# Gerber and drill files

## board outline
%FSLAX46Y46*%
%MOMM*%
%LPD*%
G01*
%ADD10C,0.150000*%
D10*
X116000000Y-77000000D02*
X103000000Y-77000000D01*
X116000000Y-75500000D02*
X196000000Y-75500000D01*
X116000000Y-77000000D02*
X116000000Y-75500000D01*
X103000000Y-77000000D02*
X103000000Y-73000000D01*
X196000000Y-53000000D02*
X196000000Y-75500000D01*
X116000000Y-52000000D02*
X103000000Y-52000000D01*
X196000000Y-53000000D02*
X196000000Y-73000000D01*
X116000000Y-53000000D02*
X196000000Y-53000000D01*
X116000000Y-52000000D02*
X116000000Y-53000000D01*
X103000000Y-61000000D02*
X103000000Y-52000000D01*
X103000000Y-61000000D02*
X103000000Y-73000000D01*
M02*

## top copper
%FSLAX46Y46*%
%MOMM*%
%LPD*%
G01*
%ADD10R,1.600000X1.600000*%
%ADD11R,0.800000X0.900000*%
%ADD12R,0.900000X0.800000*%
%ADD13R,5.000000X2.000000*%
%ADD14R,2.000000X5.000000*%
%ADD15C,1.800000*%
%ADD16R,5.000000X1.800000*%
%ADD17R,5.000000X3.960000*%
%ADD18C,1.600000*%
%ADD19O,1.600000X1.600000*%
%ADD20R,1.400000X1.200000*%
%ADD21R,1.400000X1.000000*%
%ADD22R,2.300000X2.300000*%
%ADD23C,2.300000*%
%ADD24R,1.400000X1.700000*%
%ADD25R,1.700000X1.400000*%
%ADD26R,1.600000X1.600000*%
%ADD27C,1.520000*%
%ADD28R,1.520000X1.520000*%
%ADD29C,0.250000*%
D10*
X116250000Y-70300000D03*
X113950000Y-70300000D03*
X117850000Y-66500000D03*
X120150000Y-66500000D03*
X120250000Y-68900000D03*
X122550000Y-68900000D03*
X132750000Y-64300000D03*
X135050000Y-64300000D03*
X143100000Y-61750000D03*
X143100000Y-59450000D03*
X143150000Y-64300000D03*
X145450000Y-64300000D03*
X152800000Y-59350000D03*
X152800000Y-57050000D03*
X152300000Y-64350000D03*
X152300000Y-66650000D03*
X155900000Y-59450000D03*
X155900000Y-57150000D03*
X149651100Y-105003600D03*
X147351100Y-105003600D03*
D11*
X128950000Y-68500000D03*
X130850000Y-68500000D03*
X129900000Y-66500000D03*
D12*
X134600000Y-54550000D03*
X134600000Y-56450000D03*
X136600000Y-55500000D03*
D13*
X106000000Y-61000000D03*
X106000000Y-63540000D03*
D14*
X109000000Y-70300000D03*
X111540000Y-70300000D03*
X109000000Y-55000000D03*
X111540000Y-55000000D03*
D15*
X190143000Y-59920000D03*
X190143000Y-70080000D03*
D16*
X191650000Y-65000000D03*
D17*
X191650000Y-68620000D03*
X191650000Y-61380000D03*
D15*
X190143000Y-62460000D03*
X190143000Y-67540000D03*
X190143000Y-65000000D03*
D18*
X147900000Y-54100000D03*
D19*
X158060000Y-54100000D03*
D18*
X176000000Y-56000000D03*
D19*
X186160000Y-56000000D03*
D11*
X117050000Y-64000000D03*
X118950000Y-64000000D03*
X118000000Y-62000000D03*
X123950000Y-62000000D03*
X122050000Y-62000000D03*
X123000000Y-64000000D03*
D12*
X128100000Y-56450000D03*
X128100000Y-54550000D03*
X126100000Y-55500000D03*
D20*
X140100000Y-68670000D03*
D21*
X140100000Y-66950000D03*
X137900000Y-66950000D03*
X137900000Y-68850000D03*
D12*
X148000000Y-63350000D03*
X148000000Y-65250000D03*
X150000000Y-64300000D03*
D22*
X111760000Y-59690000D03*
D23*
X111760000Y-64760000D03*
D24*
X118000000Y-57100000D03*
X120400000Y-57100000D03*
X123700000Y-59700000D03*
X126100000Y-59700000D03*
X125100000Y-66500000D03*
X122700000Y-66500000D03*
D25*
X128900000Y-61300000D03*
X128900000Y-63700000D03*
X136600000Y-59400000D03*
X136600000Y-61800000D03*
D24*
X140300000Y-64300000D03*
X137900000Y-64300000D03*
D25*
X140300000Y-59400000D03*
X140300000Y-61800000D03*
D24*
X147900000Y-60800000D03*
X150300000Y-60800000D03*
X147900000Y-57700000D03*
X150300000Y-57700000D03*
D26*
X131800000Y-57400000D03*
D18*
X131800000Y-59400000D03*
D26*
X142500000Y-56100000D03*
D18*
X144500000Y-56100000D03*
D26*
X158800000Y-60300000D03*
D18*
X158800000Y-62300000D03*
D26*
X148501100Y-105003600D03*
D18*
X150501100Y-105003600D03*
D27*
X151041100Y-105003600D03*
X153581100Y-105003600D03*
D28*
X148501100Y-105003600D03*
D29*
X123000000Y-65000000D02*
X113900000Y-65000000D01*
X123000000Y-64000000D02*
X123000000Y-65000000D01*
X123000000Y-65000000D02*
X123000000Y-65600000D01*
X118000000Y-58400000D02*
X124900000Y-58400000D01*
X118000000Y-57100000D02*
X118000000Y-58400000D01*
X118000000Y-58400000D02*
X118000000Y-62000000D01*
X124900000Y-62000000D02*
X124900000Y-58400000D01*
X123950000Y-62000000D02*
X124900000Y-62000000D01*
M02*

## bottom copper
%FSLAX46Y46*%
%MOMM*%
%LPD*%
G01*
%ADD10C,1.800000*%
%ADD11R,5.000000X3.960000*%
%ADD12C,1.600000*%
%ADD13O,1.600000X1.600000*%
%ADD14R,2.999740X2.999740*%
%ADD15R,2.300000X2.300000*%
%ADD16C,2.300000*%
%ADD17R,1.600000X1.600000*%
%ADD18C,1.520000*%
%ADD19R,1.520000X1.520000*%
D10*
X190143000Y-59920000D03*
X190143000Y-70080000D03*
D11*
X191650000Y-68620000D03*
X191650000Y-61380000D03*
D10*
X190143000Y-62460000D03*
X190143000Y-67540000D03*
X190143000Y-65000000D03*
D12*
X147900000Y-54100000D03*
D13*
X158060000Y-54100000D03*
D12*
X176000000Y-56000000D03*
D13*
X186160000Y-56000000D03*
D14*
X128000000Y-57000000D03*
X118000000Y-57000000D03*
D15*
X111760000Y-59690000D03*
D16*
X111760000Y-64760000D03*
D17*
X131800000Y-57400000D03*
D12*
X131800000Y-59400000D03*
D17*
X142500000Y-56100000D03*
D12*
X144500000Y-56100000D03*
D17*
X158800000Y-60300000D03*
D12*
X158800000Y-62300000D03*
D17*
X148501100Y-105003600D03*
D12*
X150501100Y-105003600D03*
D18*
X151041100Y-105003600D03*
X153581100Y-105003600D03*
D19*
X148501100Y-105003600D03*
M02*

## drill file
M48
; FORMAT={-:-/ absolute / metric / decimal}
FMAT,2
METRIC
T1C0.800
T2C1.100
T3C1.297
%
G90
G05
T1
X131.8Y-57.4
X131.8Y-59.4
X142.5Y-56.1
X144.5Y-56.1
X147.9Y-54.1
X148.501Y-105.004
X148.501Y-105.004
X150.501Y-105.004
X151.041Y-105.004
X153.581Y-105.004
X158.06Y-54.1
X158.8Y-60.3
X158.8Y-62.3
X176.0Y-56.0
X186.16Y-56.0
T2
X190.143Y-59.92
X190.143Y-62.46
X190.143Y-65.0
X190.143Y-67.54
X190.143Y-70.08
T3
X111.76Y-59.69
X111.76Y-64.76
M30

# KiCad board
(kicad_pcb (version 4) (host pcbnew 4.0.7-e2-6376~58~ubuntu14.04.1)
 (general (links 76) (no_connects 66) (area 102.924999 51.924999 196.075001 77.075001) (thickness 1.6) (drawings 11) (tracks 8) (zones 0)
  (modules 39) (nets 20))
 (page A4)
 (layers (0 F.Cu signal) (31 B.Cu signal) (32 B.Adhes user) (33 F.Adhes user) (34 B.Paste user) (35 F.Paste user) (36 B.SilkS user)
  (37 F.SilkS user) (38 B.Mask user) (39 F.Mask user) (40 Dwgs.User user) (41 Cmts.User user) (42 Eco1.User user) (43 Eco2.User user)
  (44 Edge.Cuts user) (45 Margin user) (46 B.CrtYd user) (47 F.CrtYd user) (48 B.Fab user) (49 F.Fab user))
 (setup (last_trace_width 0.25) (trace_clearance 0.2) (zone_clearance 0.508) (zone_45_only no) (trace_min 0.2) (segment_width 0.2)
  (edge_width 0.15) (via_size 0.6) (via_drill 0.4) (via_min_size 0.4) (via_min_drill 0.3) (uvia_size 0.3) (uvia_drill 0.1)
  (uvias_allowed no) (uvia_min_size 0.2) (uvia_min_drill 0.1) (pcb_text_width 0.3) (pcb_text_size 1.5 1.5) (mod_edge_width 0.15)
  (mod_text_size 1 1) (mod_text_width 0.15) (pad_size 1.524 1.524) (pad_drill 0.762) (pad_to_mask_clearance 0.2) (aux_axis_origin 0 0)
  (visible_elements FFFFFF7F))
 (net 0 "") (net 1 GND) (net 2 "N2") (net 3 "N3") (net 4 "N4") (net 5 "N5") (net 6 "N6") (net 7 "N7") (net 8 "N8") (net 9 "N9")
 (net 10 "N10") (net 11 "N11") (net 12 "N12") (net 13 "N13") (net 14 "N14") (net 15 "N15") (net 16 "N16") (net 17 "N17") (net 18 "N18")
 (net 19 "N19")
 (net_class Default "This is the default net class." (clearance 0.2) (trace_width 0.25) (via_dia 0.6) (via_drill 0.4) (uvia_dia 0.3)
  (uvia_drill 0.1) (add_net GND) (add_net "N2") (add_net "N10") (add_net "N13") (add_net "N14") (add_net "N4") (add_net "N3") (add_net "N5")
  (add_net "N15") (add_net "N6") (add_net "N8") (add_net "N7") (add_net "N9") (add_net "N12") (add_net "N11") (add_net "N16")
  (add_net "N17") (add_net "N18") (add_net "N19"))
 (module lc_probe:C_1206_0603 (layer F.Cu) (at 115.1 70.3)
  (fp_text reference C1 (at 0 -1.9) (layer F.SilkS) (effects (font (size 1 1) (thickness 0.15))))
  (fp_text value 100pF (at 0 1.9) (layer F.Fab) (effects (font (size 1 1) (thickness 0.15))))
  (pad 2 smd rect (at 1.15 0) (size 1.6 1.6) (layers F.Cu F.Paste F.Mask) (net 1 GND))
  (pad 1 smd rect (at -1.15 0) (size 1.6 1.6) (layers F.Cu F.Paste F.Mask) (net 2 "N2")))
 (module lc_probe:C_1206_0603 (layer F.Cu) (at 119 66.5 180)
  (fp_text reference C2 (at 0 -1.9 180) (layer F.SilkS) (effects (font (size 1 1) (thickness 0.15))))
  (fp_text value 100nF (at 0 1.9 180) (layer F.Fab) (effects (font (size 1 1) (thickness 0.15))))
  (pad 2 smd rect (at 1.15 0 180) (size 1.6 1.6) (layers F.Cu F.Paste F.Mask) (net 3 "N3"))
  (pad 1 smd rect (at -1.15 0 180) (size 1.6 1.6) (layers F.Cu F.Paste F.Mask) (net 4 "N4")))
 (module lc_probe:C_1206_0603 (layer F.Cu) (at 121.4 68.9 180)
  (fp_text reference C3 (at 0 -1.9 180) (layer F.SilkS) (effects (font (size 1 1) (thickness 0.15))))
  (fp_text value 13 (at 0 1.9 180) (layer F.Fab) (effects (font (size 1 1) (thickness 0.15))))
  (pad 2 smd rect (at 1.15 0 180) (size 1.6 1.6) (layers F.Cu F.Paste F.Mask) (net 3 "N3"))
  (pad 1 smd rect (at -1.15 0 180) (size 1.6 1.6) (layers F.Cu F.Paste F.Mask) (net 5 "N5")))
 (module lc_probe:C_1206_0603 (layer F.Cu) (at 133.9 64.3 180)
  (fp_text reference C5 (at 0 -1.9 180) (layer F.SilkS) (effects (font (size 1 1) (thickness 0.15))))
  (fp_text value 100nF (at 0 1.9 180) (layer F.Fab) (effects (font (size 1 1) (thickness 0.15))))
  (pad 2 smd rect (at 1.15 0 180) (size 1.6 1.6) (layers F.Cu F.Paste F.Mask) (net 1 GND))
  (pad 1 smd rect (at -1.15 0 180) (size 1.6 1.6) (layers F.Cu F.Paste F.Mask) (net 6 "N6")))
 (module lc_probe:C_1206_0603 (layer F.Cu) (at 143.1 60.6 270)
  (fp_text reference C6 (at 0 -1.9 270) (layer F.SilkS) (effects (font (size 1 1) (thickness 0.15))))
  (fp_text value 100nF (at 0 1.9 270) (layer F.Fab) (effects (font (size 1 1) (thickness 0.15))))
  (pad 2 smd rect (at 1.15 0 270) (size 1.6 1.6) (layers F.Cu F.Paste F.Mask) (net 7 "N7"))
  (pad 1 smd rect (at -1.15 0 270) (size 1.6 1.6) (layers F.Cu F.Paste F.Mask) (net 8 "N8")))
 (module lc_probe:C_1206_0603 (layer F.Cu) (at 144.3 64.3 180)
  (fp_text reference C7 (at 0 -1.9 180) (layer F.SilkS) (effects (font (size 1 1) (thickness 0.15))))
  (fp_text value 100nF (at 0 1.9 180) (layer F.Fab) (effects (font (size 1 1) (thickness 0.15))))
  (pad 2 smd rect (at 1.15 0 180) (size 1.6 1.6) (layers F.Cu F.Paste F.Mask) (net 7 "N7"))
  (pad 1 smd rect (at -1.15 0 180) (size 1.6 1.6) (layers F.Cu F.Paste F.Mask) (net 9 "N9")))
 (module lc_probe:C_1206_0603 (layer F.Cu) (at 152.8 58.2 270)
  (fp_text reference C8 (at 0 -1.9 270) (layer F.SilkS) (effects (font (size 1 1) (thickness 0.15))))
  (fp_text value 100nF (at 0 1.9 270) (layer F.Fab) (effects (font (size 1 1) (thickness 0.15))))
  (pad 2 smd rect (at 1.15 0 270) (size 1.6 1.6) (layers F.Cu F.Paste F.Mask) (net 1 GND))
  (pad 1 smd rect (at -1.15 0 270) (size 1.6 1.6) (layers F.Cu F.Paste F.Mask) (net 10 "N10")))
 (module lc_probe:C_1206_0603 (layer F.Cu) (at 152.3 65.5 90)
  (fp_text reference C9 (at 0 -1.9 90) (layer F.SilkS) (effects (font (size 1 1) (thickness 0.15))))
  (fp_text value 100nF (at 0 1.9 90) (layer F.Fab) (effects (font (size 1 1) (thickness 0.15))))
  (pad 2 smd rect (at 1.15 0 90) (size 1.6 1.6) (layers F.Cu F.Paste F.Mask) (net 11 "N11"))
  (pad 1 smd rect (at -1.15 0 90) (size 1.6 1.6) (layers F.Cu F.Paste F.Mask) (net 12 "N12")))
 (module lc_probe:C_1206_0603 (layer F.Cu) (at 155.9 58.3 270)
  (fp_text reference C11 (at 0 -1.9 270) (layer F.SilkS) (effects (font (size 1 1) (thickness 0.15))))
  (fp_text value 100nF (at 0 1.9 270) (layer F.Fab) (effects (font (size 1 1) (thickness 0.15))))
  (pad 2 smd rect (at 1.15 0 270) (size 1.6 1.6) (layers F.Cu F.Paste F.Mask) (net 1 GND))
  (pad 1 smd rect (at -1.15 0 270) (size 1.6 1.6) (layers F.Cu F.Paste F.Mask) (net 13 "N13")))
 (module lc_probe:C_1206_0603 (layer F.Cu) (at 148.5011 105.0036)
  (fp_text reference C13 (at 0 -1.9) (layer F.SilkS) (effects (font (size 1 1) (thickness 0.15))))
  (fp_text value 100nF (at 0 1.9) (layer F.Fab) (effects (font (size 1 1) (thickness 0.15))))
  (pad 2 smd rect (at 1.15 0) (size 1.6 1.6) (layers F.Cu F.Paste F.Mask) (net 1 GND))
  (pad 1 smd rect (at -1.15 0) (size 1.6 1.6) (layers F.Cu F.Paste F.Mask) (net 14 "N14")))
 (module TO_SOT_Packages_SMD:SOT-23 (layer F.Cu) (at 129.9 67.5 90)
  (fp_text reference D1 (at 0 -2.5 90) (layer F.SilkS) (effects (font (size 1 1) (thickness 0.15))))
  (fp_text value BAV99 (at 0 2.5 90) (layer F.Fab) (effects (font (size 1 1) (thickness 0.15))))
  (pad 1 smd rect (at -1 -0.95 90) (size 0.9 0.8) (layers F.Cu F.Paste F.Mask) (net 1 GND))
  (pad 2 smd rect (at -1 0.95 90) (size 0.9 0.8) (layers F.Cu F.Paste F.Mask) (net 1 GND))
  (pad 3 smd rect (at 1 0 90) (size 0.9 0.8) (layers F.Cu F.Paste F.Mask) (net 5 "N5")))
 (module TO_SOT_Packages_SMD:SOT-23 (layer F.Cu) (at 135.6 55.5)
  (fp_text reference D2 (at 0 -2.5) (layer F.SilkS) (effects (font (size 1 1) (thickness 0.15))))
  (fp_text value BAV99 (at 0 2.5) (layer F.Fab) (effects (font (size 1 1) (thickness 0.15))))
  (pad 1 smd rect (at -1 -0.95) (size 0.9 0.8) (layers F.Cu F.Paste F.Mask) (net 10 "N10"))
  (pad 2 smd rect (at -1 0.95) (size 0.9 0.8) (layers F.Cu F.Paste F.Mask) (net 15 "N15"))
  (pad 3 smd rect (at 1 0) (size 0.9 0.8) (layers F.Cu F.Paste F.Mask) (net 8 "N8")))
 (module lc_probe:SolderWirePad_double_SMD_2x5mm (layer F.Cu) (at 106 61 270)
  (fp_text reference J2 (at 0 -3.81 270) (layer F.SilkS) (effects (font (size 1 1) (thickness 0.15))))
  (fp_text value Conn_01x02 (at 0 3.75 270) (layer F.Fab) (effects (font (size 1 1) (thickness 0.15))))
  (pad 1 smd rect (at 0 0 270) (size 2 5) (layers F.Cu F.Paste F.Mask) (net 3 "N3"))
  (pad 2 smd rect (at 2.54 0 270) (size 2 5) (layers F.Cu F.Paste F.Mask) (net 1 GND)))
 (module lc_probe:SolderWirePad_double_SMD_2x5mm (layer F.Cu) (at 109 70.3)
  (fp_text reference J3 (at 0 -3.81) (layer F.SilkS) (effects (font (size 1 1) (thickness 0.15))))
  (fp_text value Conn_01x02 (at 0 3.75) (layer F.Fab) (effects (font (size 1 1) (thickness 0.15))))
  (pad 1 smd rect (at 0 0) (size 2 5) (layers F.Cu F.Paste F.Mask) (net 3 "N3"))
  (pad 2 smd rect (at 2.54 0) (size 2 5) (layers F.Cu F.Paste F.Mask) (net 2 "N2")))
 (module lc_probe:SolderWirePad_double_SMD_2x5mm (layer F.Cu) (at 109 55)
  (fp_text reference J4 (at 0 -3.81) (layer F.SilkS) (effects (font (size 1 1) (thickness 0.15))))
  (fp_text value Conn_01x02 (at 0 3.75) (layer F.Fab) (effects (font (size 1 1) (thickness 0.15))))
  (pad 1 smd rect (at 0 0) (size 2 5) (layers F.Cu F.Paste F.Mask) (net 3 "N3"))
  (pad 2 smd rect (at 2.54 0) (size 2 5) (layers F.Cu F.Paste F.Mask) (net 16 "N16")))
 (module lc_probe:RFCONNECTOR (layer F.Cu) (at 189 65 180)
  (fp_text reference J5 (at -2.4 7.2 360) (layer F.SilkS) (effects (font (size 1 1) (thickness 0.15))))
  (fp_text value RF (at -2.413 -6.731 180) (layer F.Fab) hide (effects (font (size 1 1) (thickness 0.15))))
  (pad 2 thru_hole circle (at -1.143 5.08 180) (size 1.8 1.8) (drill 1.1) (layers *.Cu *.Mask F.SilkS) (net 1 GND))
  (pad 2 thru_hole circle (at -1.143 -5.08 180) (size 1.8 1.8) (drill 1.1) (layers *.Cu *.Mask F.SilkS) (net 1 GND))
  (pad 1 smd rect (at -2.65 0 180) (size 5 1.8) (layers F.Cu F.Paste F.Mask) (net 12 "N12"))
  (pad 2 smd rect (at -2.65 -3.62 180) (size 5 3.96) (layers F.Cu F.Paste F.Mask) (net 1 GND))
  (pad 2 smd rect (at -2.65 3.62 180) (size 5 3.96) (layers F.Cu F.Paste F.Mask) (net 1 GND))
  (pad 2 smd rect (at -2.65 -3.62 180) (size 5 3.96) (layers B.Cu B.Paste B.Mask) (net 1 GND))
  (pad 2 smd rect (at -2.65 3.62 180) (size 5 3.96) (layers B.Cu B.Paste B.Mask) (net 1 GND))
  (pad 2 thru_hole circle (at -1.143 2.54 180) (size 1.8 1.8) (drill 1.1) (layers *.Cu *.Mask F.SilkS) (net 1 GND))
  (pad 2 thru_hole circle (at -1.143 -2.54 180) (size 1.8 1.8) (drill 1.1) (layers *.Cu *.Mask F.SilkS) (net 1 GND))
  (pad 1 thru_hole circle (at -1.143 0 180) (size 1.8 1.8) (drill 1.1) (layers *.Cu *.Mask F.SilkS) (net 12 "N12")))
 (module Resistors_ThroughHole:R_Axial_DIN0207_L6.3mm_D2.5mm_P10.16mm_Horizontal (layer B.Cu) (at 147.9 54.1)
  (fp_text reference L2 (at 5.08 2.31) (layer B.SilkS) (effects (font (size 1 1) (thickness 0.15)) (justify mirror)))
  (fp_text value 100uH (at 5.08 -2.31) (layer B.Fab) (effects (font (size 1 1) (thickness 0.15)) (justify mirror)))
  (pad 1 thru_hole circle (at 0 0) (size 1.6 1.6) (drill 0.8) (layers *.Cu *.Mask) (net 10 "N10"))
  (pad 2 thru_hole oval (at 10.16 0) (size 1.6 1.6) (drill 0.8) (layers *.Cu *.Mask) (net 13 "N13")))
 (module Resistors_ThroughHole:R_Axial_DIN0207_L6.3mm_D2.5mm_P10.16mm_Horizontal (layer B.Cu) (at 176 56)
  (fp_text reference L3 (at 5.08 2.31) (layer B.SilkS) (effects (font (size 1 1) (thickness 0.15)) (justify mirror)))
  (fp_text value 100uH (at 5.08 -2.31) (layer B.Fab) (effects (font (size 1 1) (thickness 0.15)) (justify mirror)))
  (pad 1 thru_hole circle (at 0 0) (size 1.6 1.6) (drill 0.8) (layers *.Cu *.Mask) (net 14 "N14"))
  (pad 2 thru_hole oval (at 10.16 0) (size 1.6 1.6) (drill 0.8) (layers *.Cu *.Mask) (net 12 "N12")))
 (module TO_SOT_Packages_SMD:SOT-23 (layer F.Cu) (at 118 63 90)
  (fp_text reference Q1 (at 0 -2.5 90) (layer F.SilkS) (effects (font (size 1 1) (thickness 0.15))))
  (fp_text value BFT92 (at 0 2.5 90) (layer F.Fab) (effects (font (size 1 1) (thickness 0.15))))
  (pad 1 smd rect (at -1 -0.95 90) (size 0.9 0.8) (layers F.Cu F.Paste F.Mask) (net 3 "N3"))
  (pad 2 smd rect (at -1 0.95 90) (size 0.9 0.8) (layers F.Cu F.Paste F.Mask) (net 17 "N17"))
  (pad 3 smd rect (at 1 0 90) (size 0.9 0.8) (layers F.Cu F.Paste F.Mask) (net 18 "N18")))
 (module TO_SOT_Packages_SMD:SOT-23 (layer F.Cu) (at 123 63 270)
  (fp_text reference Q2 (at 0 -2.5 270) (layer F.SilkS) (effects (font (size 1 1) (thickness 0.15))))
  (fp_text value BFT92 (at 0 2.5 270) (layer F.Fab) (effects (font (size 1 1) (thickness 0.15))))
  (pad 1 smd rect (at -1 -0.95 270) (size 0.9 0.8) (layers F.Cu F.Paste F.Mask) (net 18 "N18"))
  (pad 2 smd rect (at -1 0.95 270) (size 0.9 0.8) (layers F.Cu F.Paste F.Mask) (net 17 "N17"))
  (pad 3 smd rect (at 1 0 270) (size 0.9 0.8) (layers F.Cu F.Paste F.Mask) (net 3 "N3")))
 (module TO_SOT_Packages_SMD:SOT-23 (layer F.Cu) (at 127.1 55.5 180)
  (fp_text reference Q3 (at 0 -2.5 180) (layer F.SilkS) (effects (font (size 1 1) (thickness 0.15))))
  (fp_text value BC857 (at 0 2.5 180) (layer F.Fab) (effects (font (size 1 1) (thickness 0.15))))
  (pad 1 smd rect (at -1 -0.95 180) (size 0.9 0.8) (layers F.Cu F.Paste F.Mask) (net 15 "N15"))
  (pad 2 smd rect (at -1 0.95 180) (size 0.9 0.8) (layers F.Cu F.Paste F.Mask) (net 10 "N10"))
  (pad 3 smd rect (at 1 0 180) (size 0.9 0.8) (layers F.Cu F.Paste F.Mask) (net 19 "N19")))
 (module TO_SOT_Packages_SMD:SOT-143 (layer F.Cu) (at 139 67.9 180)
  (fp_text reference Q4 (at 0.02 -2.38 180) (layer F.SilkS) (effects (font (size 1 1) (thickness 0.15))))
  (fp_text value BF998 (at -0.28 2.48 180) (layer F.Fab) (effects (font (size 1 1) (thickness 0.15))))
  (pad 1 smd rect (at -1.1 -0.77 90) (size 1.2 1.4) (layers F.Cu F.Paste F.Mask) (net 1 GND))
  (pad 2 smd rect (at -1.1 0.95 90) (size 1 1.4) (layers F.Cu F.Paste F.Mask) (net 7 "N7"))
  (pad 3 smd rect (at 1.1 0.95 90) (size 1 1.4) (layers F.Cu F.Paste F.Mask) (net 6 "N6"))
  (pad 4 smd rect (at 1.1 -0.95 90) (size 1 1.4) (layers F.Cu F.Paste F.Mask) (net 5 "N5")))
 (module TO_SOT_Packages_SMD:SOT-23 (layer F.Cu) (at 149 64.3)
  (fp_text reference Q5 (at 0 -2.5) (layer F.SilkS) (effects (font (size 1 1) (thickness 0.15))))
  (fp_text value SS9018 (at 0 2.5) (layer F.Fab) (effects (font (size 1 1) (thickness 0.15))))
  (pad 1 smd rect (at -1 -0.95) (size 0.9 0.8) (layers F.Cu F.Paste F.Mask) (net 9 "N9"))
  (pad 2 smd rect (at -1 0.95) (size 0.9 0.8) (layers F.Cu F.Paste F.Mask) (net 1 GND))
  (pad 3 smd rect (at 1 0) (size 0.9 0.8) (layers F.Cu F.Paste F.Mask) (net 11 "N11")))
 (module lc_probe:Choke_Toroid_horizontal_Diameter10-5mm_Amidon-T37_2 (layer B.Cu) (at 123 62 180)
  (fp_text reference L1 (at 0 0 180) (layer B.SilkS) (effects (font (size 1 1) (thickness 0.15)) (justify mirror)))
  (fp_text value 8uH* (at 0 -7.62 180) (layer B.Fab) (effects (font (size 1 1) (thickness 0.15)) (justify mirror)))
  (pad 1 smd rect (at -5 5 180) (size 2.99974 2.99974) (layers B.Cu B.Paste B.Mask) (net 1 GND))
  (pad 2 smd rect (at 5 5 180) (size 2.99974 2.99974) (layers B.Cu B.Paste B.Mask) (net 16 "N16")))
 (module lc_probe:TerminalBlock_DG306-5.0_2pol (layer B.Cu) (at 111.76 58.42 270)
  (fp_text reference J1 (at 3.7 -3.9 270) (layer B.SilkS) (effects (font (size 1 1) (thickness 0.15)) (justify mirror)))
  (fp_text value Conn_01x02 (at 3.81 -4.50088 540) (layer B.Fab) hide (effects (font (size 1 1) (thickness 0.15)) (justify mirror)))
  (pad 1 thru_hole rect (at 1.27 0 90) (size 2.3 2.3) (drill 1.29728) (layers *.Cu *.Mask) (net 3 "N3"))
  (pad 2 thru_hole circle (at 6.34 0 90) (size 2.3 2.3) (drill 1.29728) (layers *.Cu *.Mask) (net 1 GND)))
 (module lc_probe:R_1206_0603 (layer F.Cu) (at 119.2 57.1)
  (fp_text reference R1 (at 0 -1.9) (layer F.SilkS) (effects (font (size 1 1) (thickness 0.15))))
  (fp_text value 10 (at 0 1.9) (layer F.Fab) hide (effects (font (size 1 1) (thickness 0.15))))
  (pad 1 smd rect (at -1.2 0 90) (size 1.7 1.4) (layers F.Cu F.Paste F.Mask) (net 18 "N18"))
  (pad 2 smd rect (at 1.2 0) (size 1.4 1.7) (layers F.Cu F.Paste F.Mask) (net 1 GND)))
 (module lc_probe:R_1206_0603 (layer F.Cu) (at 124.9 59.7)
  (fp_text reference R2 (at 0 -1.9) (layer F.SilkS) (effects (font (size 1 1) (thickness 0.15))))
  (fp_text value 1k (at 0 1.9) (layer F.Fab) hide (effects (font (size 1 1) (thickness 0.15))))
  (pad 1 smd rect (at -1.2 0 90) (size 1.7 1.4) (layers F.Cu F.Paste F.Mask) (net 17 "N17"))
  (pad 2 smd rect (at 1.2 0) (size 1.4 1.7) (layers F.Cu F.Paste F.Mask) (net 19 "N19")))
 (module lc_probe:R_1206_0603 (layer F.Cu) (at 123.9 66.5 180)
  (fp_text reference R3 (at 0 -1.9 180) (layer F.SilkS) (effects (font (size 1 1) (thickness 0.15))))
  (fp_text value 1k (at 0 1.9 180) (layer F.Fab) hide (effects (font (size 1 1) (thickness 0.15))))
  (pad 1 smd rect (at -1.2 0 270) (size 1.7 1.4) (layers F.Cu F.Paste F.Mask) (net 5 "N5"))
  (pad 2 smd rect (at 1.2 0 180) (size 1.4 1.7) (layers F.Cu F.Paste F.Mask) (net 4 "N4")))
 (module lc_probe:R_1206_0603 (layer F.Cu) (at 128.9 62.5 270)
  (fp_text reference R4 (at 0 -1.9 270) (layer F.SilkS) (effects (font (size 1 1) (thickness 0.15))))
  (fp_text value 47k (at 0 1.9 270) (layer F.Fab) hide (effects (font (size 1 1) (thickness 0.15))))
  (pad 1 smd rect (at -1.2 0) (size 1.7 1.4) (layers F.Cu F.Paste F.Mask) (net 15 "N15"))
  (pad 2 smd rect (at 1.2 0 270) (size 1.4 1.7) (layers F.Cu F.Paste F.Mask) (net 1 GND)))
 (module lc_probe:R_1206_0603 (layer F.Cu) (at 136.6 60.6 270)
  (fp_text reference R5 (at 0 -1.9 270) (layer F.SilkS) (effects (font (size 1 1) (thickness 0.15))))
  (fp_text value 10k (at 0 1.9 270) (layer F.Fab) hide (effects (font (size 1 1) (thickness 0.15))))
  (pad 1 smd rect (at -1.2 0) (size 1.7 1.4) (layers F.Cu F.Paste F.Mask) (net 10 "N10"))
  (pad 2 smd rect (at 1.2 0 270) (size 1.4 1.7) (layers F.Cu F.Paste F.Mask) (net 6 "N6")))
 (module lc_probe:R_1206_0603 (layer F.Cu) (at 139.1 64.3 180)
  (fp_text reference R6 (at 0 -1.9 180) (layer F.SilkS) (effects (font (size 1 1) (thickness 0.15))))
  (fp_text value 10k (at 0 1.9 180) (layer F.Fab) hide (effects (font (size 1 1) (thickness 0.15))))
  (pad 1 smd rect (at -1.2 0 270) (size 1.7 1.4) (layers F.Cu F.Paste F.Mask) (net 7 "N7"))
  (pad 2 smd rect (at 1.2 0 180) (size 1.4 1.7) (layers F.Cu F.Paste F.Mask) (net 6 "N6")))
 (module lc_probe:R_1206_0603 (layer F.Cu) (at 140.3 60.6 270)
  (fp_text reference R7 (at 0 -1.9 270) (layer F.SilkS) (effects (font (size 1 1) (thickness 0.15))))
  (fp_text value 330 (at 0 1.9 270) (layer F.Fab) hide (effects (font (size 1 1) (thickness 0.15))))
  (pad 1 smd rect (at -1.2 0) (size 1.7 1.4) (layers F.Cu F.Paste F.Mask) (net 10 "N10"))
  (pad 2 smd rect (at 1.2 0 270) (size 1.4 1.7) (layers F.Cu F.Paste F.Mask) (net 7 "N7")))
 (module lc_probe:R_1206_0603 (layer F.Cu) (at 149.1 60.8)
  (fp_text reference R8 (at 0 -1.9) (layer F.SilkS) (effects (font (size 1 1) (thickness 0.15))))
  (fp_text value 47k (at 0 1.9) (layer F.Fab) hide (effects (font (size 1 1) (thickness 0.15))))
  (pad 1 smd rect (at -1.2 0 90) (size 1.7 1.4) (layers F.Cu F.Paste F.Mask) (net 9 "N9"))
  (pad 2 smd rect (at 1.2 0) (size 1.4 1.7) (layers F.Cu F.Paste F.Mask) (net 11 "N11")))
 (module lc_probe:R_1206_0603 (layer F.Cu) (at 149.1 57.7)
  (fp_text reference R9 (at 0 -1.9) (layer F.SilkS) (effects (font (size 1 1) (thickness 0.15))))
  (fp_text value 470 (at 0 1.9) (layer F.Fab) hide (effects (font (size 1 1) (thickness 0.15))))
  (pad 1 smd rect (at -1.2 0 90) (size 1.7 1.4) (layers F.Cu F.Paste F.Mask) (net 10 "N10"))
  (pad 2 smd rect (at 1.2 0) (size 1.4 1.7) (layers F.Cu F.Paste F.Mask) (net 11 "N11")))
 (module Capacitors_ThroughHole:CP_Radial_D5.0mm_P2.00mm (layer F.Cu) (at 131.8 57.4 270)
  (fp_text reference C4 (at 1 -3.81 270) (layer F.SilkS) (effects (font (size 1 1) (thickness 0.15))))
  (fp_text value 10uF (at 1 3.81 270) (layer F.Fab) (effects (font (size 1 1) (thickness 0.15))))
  (pad 1 thru_hole rect (at 0 0 270) (size 1.6 1.6) (drill 0.8) (layers *.Cu *.Mask) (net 10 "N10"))
  (pad 2 thru_hole circle (at 2 0 270) (size 1.6 1.6) (drill 0.8) (layers *.Cu *.Mask) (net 15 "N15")))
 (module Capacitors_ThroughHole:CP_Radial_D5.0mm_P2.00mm (layer F.Cu) (at 142.5 56.1)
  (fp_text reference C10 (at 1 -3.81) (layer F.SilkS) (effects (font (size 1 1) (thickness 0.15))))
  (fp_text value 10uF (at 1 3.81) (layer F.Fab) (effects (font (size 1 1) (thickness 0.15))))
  (pad 1 thru_hole rect (at 0 0) (size 1.6 1.6) (drill 0.8) (layers *.Cu *.Mask) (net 10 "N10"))
  (pad 2 thru_hole circle (at 2 0) (size 1.6 1.6) (drill 0.8) (layers *.Cu *.Mask) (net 1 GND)))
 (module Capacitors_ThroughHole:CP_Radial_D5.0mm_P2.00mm (layer F.Cu) (at 158.8 60.3 270)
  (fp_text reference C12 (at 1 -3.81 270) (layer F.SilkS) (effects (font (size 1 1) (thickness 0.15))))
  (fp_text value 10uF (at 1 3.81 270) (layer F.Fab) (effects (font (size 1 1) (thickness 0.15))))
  (pad 1 thru_hole rect (at 0 0 270) (size 1.6 1.6) (drill 0.8) (layers *.Cu *.Mask) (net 13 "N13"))
  (pad 2 thru_hole circle (at 2 0 270) (size 1.6 1.6) (drill 0.8) (layers *.Cu *.Mask) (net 1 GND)))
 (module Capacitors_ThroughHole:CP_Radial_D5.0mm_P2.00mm (layer F.Cu) (at 148.5011 105.0036)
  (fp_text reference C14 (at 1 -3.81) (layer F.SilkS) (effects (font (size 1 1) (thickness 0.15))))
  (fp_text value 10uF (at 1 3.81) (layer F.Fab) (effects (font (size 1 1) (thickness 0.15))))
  (pad 1 thru_hole rect (at 0 0) (size 1.6 1.6) (drill 0.8) (layers *.Cu *.Mask) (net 14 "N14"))
  (pad 2 thru_hole circle (at 2 0) (size 1.6 1.6) (drill 0.8) (layers *.Cu *.Mask) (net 1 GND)))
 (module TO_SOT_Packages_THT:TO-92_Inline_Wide (layer F.Cu) (at 148.5011 105.0036)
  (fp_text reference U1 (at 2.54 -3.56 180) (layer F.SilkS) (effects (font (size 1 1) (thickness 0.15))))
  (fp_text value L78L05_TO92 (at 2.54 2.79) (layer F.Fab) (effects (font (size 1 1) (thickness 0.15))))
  (pad 2 thru_hole circle (at 2.54 0 90) (size 1.52 1.52) (drill 0.8) (layers *.Cu *.Mask) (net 1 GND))
  (pad 3 thru_hole circle (at 5.08 0 90) (size 1.52 1.52) (drill 0.8) (layers *.Cu *.Mask) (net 14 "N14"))
  (pad 1 thru_hole rect (at 0 0 90) (size 1.52 1.52) (drill 0.8) (layers *.Cu *.Mask) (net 13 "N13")))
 (gr_line (start 116 77) (end 103 77) (angle 90) (layer Edge.Cuts) (width 0.15))
 (gr_line (start 116 75.5) (end 196 75.5) (angle 90) (layer Edge.Cuts) (width 0.15))
 (gr_line (start 116 77) (end 116 75.5) (angle 90) (layer Edge.Cuts) (width 0.15))
 (gr_line (start 103 77) (end 103 73) (angle 90) (layer Edge.Cuts) (width 0.15))
 (gr_line (start 196 53) (end 196 75.5) (angle 90) (layer Edge.Cuts) (width 0.15))
 (gr_line (start 116 52) (end 103 52) (angle 90) (layer Edge.Cuts) (width 0.15))
 (gr_line (start 196 53) (end 196 73) (angle 90) (layer Edge.Cuts) (width 0.15))
 (gr_line (start 116 53) (end 196 53) (angle 90) (layer Edge.Cuts) (width 0.15))
 (gr_line (start 116 52) (end 116 53) (angle 90) (layer Edge.Cuts) (width 0.15))
 (gr_line (start 103 61) (end 103 52) (angle 90) (layer Edge.Cuts) (width 0.15))
 (gr_line (start 103 61) (end 103 73) (angle 90) (layer Edge.Cuts) (width 0.15))
 (segment (start 123 65) (end 113.9 65) (width 0.25) (layer F.Cu) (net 3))
 (segment (start 123 64) (end 123 65) (width 0.25) (layer F.Cu) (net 3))
 (segment (start 123 65) (end 123 65.6) (width 0.25) (layer F.Cu) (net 3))
 (segment (start 118 58.4) (end 124.9 58.4) (width 0.25) (layer F.Cu) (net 18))
 (segment (start 118 57.1) (end 118 58.4) (width 0.25) (layer F.Cu) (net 18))
 (segment (start 118 58.4) (end 118 62) (width 0.25) (layer F.Cu) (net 18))
 (segment (start 124.9 62) (end 124.9 58.4) (width 0.25) (layer F.Cu) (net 18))
 (segment (start 123.95 62) (end 124.9 62) (width 0.25) (layer F.Cu) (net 18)))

